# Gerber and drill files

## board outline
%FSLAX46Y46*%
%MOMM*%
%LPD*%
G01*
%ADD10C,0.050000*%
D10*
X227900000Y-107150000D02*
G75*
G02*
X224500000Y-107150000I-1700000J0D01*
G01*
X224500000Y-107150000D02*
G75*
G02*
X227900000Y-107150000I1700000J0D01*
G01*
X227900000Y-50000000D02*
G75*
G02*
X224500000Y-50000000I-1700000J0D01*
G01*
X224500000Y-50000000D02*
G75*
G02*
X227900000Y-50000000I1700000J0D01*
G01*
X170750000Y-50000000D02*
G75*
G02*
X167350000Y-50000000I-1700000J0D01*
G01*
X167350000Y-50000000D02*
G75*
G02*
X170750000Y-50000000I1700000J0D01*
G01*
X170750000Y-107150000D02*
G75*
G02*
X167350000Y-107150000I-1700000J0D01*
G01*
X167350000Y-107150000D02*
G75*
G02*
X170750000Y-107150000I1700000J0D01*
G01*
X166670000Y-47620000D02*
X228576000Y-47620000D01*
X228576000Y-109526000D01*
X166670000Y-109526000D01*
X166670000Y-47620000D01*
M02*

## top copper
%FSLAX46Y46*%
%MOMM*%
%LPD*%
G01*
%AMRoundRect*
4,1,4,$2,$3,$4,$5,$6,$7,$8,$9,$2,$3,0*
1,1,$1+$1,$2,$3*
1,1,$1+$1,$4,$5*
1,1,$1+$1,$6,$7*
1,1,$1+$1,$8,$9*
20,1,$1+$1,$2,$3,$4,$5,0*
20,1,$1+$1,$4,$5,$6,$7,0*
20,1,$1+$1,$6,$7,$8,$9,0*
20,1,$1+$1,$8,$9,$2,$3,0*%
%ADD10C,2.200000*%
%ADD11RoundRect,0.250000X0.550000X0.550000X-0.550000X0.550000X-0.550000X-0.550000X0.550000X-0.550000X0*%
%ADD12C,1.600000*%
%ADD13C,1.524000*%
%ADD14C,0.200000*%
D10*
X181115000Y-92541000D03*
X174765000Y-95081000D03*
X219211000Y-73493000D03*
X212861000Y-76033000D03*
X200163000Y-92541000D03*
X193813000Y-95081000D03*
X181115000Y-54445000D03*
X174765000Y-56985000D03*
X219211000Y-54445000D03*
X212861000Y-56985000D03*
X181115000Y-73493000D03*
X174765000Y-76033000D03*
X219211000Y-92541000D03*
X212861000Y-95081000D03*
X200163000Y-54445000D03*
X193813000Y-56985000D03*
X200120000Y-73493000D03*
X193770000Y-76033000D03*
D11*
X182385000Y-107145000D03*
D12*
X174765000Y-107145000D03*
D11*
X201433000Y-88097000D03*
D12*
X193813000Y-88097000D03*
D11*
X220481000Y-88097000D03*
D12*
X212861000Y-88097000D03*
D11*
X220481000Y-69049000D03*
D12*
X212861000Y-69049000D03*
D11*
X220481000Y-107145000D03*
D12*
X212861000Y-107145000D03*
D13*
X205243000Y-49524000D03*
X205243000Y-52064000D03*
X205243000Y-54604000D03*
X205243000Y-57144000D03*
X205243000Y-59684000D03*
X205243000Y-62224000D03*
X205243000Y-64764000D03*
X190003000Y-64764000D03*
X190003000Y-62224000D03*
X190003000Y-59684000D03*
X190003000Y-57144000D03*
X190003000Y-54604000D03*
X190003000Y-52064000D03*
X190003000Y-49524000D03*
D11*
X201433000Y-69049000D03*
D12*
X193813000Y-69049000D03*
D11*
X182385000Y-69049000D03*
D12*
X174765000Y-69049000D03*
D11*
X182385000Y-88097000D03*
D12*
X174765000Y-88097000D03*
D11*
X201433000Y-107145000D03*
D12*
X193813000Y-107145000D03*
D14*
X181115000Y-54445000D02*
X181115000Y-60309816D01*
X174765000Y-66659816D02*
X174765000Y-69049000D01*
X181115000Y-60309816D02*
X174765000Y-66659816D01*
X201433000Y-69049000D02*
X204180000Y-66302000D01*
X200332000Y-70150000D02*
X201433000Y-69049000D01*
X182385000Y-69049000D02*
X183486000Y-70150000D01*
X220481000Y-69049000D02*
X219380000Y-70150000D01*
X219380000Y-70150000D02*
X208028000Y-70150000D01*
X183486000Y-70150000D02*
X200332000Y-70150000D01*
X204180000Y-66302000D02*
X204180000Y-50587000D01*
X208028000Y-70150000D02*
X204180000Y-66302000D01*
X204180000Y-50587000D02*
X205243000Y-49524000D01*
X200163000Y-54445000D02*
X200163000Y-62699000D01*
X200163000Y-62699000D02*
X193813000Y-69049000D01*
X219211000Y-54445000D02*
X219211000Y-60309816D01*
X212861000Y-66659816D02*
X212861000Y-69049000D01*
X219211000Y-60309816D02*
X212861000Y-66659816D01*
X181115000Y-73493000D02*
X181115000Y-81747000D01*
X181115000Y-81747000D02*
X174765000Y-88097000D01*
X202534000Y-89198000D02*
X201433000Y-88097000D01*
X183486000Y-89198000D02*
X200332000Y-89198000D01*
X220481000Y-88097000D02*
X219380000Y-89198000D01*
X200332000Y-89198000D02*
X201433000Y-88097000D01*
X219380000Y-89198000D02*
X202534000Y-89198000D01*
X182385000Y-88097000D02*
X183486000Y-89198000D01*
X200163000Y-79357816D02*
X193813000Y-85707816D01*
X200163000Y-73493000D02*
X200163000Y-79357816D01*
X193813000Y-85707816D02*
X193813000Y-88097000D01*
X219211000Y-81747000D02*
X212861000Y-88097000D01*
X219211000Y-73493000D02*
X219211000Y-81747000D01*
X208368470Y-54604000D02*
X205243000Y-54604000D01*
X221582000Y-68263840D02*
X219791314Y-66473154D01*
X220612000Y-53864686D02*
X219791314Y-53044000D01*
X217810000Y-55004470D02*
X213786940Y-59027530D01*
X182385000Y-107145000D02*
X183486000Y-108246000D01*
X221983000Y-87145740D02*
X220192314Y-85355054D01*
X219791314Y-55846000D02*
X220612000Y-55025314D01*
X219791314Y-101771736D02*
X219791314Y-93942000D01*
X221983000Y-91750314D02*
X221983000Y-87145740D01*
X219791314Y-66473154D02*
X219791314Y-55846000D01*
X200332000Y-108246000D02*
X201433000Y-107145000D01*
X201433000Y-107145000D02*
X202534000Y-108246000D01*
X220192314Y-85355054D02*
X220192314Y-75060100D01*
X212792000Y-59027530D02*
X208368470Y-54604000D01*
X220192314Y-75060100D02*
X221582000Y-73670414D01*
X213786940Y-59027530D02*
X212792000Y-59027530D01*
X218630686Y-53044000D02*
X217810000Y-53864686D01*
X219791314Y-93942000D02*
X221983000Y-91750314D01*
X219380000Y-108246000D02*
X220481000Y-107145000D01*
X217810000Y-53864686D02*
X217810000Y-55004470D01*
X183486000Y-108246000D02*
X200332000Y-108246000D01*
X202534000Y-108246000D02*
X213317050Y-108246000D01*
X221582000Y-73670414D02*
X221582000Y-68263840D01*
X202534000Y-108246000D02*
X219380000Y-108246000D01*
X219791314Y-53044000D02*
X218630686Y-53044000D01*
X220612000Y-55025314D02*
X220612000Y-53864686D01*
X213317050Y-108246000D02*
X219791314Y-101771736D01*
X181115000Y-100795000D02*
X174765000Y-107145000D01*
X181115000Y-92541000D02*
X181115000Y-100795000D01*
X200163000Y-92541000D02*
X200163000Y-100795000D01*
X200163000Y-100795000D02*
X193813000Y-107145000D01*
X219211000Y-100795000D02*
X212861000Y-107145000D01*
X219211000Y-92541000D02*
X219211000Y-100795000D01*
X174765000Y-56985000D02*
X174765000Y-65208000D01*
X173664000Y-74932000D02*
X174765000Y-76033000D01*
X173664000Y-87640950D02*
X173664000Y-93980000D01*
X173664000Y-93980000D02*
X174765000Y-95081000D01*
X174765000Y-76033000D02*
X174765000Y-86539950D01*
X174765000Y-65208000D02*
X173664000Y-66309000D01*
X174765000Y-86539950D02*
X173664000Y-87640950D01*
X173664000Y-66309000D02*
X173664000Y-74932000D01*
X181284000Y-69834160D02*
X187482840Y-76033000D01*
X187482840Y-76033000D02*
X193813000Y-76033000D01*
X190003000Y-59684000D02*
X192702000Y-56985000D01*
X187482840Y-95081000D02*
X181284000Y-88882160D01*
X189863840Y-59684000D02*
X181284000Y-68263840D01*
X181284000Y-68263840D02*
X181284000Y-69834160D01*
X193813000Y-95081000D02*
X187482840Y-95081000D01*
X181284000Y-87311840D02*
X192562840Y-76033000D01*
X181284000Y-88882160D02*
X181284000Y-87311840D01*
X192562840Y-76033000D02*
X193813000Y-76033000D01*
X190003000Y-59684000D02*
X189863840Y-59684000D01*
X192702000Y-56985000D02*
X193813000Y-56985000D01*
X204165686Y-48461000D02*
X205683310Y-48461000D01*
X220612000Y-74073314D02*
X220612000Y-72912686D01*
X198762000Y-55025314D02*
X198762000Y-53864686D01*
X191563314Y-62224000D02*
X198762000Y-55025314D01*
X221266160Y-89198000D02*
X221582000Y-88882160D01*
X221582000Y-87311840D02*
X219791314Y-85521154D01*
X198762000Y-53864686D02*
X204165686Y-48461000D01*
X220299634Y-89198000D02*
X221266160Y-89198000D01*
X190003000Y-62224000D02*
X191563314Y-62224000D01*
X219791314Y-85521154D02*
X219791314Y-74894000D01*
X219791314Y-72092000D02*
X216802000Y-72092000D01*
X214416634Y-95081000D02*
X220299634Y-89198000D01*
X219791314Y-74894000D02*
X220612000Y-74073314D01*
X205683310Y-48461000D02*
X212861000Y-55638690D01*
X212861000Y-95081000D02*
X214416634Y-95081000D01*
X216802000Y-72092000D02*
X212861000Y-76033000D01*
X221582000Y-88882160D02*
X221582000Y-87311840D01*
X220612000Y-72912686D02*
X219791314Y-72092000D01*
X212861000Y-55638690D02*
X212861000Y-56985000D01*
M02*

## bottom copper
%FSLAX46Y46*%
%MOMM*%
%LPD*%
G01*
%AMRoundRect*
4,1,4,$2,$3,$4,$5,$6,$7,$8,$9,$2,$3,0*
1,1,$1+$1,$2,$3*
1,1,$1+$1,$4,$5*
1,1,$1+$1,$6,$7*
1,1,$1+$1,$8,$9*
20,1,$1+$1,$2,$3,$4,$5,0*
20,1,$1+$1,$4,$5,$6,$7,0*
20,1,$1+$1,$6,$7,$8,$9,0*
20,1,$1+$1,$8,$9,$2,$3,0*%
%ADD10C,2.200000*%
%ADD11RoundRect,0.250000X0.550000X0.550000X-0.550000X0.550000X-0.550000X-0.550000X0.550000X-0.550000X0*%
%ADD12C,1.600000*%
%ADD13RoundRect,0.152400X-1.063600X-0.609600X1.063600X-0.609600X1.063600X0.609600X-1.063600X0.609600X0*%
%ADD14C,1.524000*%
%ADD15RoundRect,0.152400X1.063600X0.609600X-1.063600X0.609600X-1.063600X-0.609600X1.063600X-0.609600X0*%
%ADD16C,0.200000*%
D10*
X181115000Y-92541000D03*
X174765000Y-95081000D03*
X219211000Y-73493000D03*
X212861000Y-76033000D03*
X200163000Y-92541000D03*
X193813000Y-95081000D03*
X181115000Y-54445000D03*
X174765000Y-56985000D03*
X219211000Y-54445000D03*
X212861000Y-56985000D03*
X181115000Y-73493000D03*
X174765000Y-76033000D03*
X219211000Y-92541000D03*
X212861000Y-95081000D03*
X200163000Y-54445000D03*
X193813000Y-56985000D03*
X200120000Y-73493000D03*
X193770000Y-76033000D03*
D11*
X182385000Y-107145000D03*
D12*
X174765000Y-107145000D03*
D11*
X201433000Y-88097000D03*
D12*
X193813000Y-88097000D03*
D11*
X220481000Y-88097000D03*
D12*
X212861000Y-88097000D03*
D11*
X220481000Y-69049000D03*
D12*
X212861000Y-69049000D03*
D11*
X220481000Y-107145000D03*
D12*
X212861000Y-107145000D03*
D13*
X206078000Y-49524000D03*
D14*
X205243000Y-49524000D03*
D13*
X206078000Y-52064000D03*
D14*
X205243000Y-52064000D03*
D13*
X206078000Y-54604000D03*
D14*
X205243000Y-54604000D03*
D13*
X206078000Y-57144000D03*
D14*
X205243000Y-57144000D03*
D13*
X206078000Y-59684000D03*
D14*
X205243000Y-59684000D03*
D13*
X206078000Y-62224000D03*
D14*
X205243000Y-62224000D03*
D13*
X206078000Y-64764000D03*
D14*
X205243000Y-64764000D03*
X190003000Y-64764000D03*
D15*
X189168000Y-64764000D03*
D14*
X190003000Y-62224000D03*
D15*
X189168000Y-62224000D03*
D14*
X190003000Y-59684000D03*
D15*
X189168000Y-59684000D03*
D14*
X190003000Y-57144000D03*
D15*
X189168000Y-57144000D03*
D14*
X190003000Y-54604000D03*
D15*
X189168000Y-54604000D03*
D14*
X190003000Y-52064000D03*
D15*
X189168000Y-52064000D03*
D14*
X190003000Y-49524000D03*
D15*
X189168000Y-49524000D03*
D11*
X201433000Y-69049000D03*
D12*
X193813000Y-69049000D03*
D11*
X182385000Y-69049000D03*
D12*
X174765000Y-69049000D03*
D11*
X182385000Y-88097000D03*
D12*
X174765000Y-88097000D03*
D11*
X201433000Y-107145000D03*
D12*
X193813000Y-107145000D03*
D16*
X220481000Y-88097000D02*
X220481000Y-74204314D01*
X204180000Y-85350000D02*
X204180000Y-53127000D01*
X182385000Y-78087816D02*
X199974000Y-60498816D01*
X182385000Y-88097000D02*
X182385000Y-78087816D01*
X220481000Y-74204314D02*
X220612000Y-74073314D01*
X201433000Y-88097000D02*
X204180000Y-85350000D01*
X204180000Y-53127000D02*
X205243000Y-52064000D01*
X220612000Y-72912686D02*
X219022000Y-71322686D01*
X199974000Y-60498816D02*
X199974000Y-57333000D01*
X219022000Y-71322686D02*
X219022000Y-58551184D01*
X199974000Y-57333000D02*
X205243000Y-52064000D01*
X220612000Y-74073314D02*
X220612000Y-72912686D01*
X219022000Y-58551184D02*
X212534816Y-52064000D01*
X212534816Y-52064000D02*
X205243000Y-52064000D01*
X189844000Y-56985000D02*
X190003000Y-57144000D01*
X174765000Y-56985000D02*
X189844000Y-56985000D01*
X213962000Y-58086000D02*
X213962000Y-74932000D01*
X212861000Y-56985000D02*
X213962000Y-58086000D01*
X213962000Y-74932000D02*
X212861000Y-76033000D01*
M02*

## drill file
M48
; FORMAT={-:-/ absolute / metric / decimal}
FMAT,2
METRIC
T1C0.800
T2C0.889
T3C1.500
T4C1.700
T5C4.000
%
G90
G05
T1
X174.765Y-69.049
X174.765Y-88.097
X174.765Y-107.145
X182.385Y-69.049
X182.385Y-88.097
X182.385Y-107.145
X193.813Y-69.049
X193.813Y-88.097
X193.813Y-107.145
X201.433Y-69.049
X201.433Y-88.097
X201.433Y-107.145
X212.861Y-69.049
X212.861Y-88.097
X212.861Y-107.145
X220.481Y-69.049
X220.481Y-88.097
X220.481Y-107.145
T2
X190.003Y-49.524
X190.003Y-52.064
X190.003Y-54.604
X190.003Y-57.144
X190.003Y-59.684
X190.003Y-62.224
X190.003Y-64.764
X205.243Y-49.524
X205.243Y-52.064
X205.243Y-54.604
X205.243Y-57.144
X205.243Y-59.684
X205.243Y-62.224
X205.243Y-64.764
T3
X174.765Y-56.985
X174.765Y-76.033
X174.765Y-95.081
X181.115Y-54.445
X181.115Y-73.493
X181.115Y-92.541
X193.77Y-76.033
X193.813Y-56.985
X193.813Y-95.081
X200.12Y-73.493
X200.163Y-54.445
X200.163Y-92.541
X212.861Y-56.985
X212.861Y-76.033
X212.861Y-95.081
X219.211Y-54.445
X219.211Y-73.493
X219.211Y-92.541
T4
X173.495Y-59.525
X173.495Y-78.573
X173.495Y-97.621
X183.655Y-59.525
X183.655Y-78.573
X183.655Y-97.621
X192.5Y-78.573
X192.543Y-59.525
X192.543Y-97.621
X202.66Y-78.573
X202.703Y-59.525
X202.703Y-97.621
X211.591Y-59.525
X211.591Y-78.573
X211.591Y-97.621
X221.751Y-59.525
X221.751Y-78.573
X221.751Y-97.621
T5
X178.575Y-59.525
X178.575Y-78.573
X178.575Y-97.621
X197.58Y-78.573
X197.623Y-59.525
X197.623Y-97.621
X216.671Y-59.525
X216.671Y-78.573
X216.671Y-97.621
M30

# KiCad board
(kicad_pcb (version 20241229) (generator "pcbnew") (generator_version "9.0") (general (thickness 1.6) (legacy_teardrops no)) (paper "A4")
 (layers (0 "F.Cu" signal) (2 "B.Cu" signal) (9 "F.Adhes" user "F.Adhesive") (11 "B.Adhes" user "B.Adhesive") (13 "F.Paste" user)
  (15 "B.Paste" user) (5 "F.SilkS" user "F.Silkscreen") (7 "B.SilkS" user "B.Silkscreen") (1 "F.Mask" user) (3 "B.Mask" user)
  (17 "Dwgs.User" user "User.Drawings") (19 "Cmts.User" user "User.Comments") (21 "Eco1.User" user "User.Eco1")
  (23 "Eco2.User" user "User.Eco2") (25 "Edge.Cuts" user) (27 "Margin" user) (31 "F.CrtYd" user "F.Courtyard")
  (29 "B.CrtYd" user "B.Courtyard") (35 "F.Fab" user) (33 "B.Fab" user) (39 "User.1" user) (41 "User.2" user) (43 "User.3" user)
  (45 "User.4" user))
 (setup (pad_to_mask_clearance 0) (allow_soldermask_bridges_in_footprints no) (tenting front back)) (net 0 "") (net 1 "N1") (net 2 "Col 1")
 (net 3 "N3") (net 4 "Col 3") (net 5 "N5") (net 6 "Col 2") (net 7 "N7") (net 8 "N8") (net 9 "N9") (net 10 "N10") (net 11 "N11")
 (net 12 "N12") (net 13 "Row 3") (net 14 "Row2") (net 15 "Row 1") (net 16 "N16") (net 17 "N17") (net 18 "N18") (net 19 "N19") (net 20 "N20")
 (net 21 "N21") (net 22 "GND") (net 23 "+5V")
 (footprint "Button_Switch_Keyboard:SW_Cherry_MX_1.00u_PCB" (layer "F.Cu") (at 181.115 92.541)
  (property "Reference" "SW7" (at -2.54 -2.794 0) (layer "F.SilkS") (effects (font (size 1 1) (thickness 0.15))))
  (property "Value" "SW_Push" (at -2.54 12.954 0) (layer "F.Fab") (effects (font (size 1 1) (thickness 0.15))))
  (pad "" np_thru_hole circle (at -7.62 5.08) (size 1.7 1.7) (drill 1.7) (layers "*.Cu" "*.Mask"))
  (pad "" np_thru_hole circle (at -2.54 5.08) (size 4 4) (drill 4) (layers "*.Cu" "*.Mask"))
  (pad "" np_thru_hole circle (at 2.54 5.08) (size 1.7 1.7) (drill 1.7) (layers "*.Cu" "*.Mask"))
  (pad "1" thru_hole circle (at 0 0) (size 2.2 2.2) (drill 1.5) (layers "*.Cu" "*.Mask") (remove_unused_layers no) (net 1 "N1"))
  (pad "2" thru_hole circle (at -6.35 2.54) (size 2.2 2.2) (drill 1.5) (layers "*.Cu" "*.Mask") (remove_unused_layers no) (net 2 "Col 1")))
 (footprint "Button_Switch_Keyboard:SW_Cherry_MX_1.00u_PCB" (layer "F.Cu") (at 219.211 73.493)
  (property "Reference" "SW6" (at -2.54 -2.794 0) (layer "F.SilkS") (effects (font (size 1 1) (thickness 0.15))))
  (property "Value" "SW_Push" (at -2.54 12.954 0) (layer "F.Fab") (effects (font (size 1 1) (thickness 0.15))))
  (pad "" np_thru_hole circle (at -7.62 5.08) (size 1.7 1.7) (drill 1.7) (layers "*.Cu" "*.Mask"))
  (pad "" np_thru_hole circle (at -2.54 5.08) (size 4 4) (drill 4) (layers "*.Cu" "*.Mask"))
  (pad "" np_thru_hole circle (at 2.54 5.08) (size 1.7 1.7) (drill 1.7) (layers "*.Cu" "*.Mask"))
  (pad "1" thru_hole circle (at 0 0) (size 2.2 2.2) (drill 1.5) (layers "*.Cu" "*.Mask") (remove_unused_layers no) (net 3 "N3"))
  (pad "2" thru_hole circle (at -6.35 2.54) (size 2.2 2.2) (drill 1.5) (layers "*.Cu" "*.Mask") (remove_unused_layers no) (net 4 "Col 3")))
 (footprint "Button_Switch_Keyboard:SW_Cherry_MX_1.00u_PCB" (layer "F.Cu") (at 200.163 92.541)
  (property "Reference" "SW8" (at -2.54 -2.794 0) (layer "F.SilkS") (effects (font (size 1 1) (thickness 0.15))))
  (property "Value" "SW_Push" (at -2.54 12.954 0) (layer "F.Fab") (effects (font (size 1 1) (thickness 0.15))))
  (pad "" np_thru_hole circle (at -7.62 5.08) (size 1.7 1.7) (drill 1.7) (layers "*.Cu" "*.Mask"))
  (pad "" np_thru_hole circle (at -2.54 5.08) (size 4 4) (drill 4) (layers "*.Cu" "*.Mask"))
  (pad "" np_thru_hole circle (at 2.54 5.08) (size 1.7 1.7) (drill 1.7) (layers "*.Cu" "*.Mask"))
  (pad "1" thru_hole circle (at 0 0) (size 2.2 2.2) (drill 1.5) (layers "*.Cu" "*.Mask") (remove_unused_layers no) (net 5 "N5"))
  (pad "2" thru_hole circle (at -6.35 2.54) (size 2.2 2.2) (drill 1.5) (layers "*.Cu" "*.Mask") (remove_unused_layers no) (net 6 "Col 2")))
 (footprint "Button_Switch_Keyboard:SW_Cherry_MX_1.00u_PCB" (layer "F.Cu") (at 181.115 54.445)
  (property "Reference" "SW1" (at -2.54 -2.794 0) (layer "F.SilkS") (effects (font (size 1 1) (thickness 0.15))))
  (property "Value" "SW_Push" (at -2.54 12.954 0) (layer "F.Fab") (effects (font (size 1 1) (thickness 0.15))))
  (pad "" np_thru_hole circle (at -7.62 5.08) (size 1.7 1.7) (drill 1.7) (layers "*.Cu" "*.Mask"))
  (pad "" np_thru_hole circle (at -2.54 5.08) (size 4 4) (drill 4) (layers "*.Cu" "*.Mask"))
  (pad "" np_thru_hole circle (at 2.54 5.08) (size 1.7 1.7) (drill 1.7) (layers "*.Cu" "*.Mask"))
  (pad "1" thru_hole circle (at 0 0) (size 2.2 2.2) (drill 1.5) (layers "*.Cu" "*.Mask") (remove_unused_layers no) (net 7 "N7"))
  (pad "2" thru_hole circle (at -6.35 2.54) (size 2.2 2.2) (drill 1.5) (layers "*.Cu" "*.Mask") (remove_unused_layers no) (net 2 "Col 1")))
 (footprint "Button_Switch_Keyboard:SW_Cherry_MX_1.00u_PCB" (layer "F.Cu") (at 219.211 54.445)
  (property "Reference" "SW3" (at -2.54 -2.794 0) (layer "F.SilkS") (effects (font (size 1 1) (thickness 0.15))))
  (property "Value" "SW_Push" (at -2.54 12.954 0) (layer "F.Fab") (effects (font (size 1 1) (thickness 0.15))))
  (pad "" np_thru_hole circle (at -7.62 5.08) (size 1.7 1.7) (drill 1.7) (layers "*.Cu" "*.Mask"))
  (pad "" np_thru_hole circle (at -2.54 5.08) (size 4 4) (drill 4) (layers "*.Cu" "*.Mask"))
  (pad "" np_thru_hole circle (at 2.54 5.08) (size 1.7 1.7) (drill 1.7) (layers "*.Cu" "*.Mask"))
  (pad "1" thru_hole circle (at 0 0) (size 2.2 2.2) (drill 1.5) (layers "*.Cu" "*.Mask") (remove_unused_layers no) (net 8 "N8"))
  (pad "2" thru_hole circle (at -6.35 2.54) (size 2.2 2.2) (drill 1.5) (layers "*.Cu" "*.Mask") (remove_unused_layers no) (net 4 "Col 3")))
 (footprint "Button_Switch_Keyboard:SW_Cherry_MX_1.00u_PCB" (layer "F.Cu") (at 181.115 73.493)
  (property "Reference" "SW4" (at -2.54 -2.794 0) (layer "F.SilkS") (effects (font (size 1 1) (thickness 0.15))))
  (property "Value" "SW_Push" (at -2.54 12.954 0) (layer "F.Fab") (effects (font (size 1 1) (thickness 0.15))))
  (pad "" np_thru_hole circle (at -7.62 5.08) (size 1.7 1.7) (drill 1.7) (layers "*.Cu" "*.Mask"))
  (pad "" np_thru_hole circle (at -2.54 5.08) (size 4 4) (drill 4) (layers "*.Cu" "*.Mask"))
  (pad "" np_thru_hole circle (at 2.54 5.08) (size 1.7 1.7) (drill 1.7) (layers "*.Cu" "*.Mask"))
  (pad "1" thru_hole circle (at 0 0) (size 2.2 2.2) (drill 1.5) (layers "*.Cu" "*.Mask") (remove_unused_layers no) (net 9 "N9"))
  (pad "2" thru_hole circle (at -6.35 2.54) (size 2.2 2.2) (drill 1.5) (layers "*.Cu" "*.Mask") (remove_unused_layers no) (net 2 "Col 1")))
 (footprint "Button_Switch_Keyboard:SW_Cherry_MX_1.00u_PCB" (layer "F.Cu") (at 219.211 92.541)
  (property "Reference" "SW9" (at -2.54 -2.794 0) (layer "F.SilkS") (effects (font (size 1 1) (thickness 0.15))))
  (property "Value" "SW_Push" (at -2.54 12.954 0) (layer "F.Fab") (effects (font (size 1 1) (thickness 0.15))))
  (pad "" np_thru_hole circle (at -7.62 5.08) (size 1.7 1.7) (drill 1.7) (layers "*.Cu" "*.Mask"))
  (pad "" np_thru_hole circle (at -2.54 5.08) (size 4 4) (drill 4) (layers "*.Cu" "*.Mask"))
  (pad "" np_thru_hole circle (at 2.54 5.08) (size 1.7 1.7) (drill 1.7) (layers "*.Cu" "*.Mask"))
  (pad "1" thru_hole circle (at 0 0) (size 2.2 2.2) (drill 1.5) (layers "*.Cu" "*.Mask") (remove_unused_layers no) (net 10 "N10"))
  (pad "2" thru_hole circle (at -6.35 2.54) (size 2.2 2.2) (drill 1.5) (layers "*.Cu" "*.Mask") (remove_unused_layers no) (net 4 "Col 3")))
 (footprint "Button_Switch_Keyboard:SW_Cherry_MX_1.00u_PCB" (layer "F.Cu") (at 200.163 54.445)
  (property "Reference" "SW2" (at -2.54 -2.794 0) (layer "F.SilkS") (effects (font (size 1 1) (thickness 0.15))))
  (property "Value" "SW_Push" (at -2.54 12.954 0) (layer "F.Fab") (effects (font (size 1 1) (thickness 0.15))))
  (pad "" np_thru_hole circle (at -7.62 5.08) (size 1.7 1.7) (drill 1.7) (layers "*.Cu" "*.Mask"))
  (pad "" np_thru_hole circle (at -2.54 5.08) (size 4 4) (drill 4) (layers "*.Cu" "*.Mask"))
  (pad "" np_thru_hole circle (at 2.54 5.08) (size 1.7 1.7) (drill 1.7) (layers "*.Cu" "*.Mask"))
  (pad "1" thru_hole circle (at 0 0) (size 2.2 2.2) (drill 1.5) (layers "*.Cu" "*.Mask") (remove_unused_layers no) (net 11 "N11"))
  (pad "2" thru_hole circle (at -6.35 2.54) (size 2.2 2.2) (drill 1.5) (layers "*.Cu" "*.Mask") (remove_unused_layers no) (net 6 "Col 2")))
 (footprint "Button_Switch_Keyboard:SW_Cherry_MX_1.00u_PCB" (layer "F.Cu") (at 200.12 73.493)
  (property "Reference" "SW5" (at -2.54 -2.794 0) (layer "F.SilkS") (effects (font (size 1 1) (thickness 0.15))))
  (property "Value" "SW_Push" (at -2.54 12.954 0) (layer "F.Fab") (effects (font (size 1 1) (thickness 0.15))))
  (pad "" np_thru_hole circle (at -7.62 5.08) (size 1.7 1.7) (drill 1.7) (layers "*.Cu" "*.Mask"))
  (pad "" np_thru_hole circle (at -2.54 5.08) (size 4 4) (drill 4) (layers "*.Cu" "*.Mask"))
  (pad "" np_thru_hole circle (at 2.54 5.08) (size 1.7 1.7) (drill 1.7) (layers "*.Cu" "*.Mask"))
  (pad "1" thru_hole circle (at 0 0) (size 2.2 2.2) (drill 1.5) (layers "*.Cu" "*.Mask") (remove_unused_layers no) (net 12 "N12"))
  (pad "2" thru_hole circle (at -6.35 2.54) (size 2.2 2.2) (drill 1.5) (layers "*.Cu" "*.Mask") (remove_unused_layers no) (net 6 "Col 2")))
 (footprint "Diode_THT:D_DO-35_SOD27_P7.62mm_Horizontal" (layer "B.Cu") (at 182.385 107.145 180)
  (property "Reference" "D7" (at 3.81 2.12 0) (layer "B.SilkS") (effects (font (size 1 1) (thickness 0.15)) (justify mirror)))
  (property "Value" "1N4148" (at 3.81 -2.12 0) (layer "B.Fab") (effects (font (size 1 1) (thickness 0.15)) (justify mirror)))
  (pad "1" thru_hole roundrect (at 0 0 180) (size 1.6 1.6) (drill 0.8) (layers "*.Cu" "*.Mask") (remove_unused_layers no)
   (roundrect_rratio 0.15625) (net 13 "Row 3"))
  (pad "2" thru_hole circle (at 7.62 0 180) (size 1.6 1.6) (drill 0.8) (layers "*.Cu" "*.Mask") (remove_unused_layers no) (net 1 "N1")))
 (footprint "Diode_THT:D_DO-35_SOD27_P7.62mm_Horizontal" (layer "B.Cu") (at 201.433 88.097 180)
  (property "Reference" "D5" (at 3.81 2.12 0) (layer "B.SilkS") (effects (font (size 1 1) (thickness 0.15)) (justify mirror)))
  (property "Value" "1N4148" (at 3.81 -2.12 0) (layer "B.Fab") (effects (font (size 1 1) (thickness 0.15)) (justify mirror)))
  (pad "1" thru_hole roundrect (at 0 0 180) (size 1.6 1.6) (drill 0.8) (layers "*.Cu" "*.Mask") (remove_unused_layers no)
   (roundrect_rratio 0.15625) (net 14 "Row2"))
  (pad "2" thru_hole circle (at 7.62 0 180) (size 1.6 1.6) (drill 0.8) (layers "*.Cu" "*.Mask") (remove_unused_layers no) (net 12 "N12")))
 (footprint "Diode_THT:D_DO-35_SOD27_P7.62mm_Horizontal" (layer "B.Cu") (at 220.481 88.097 180)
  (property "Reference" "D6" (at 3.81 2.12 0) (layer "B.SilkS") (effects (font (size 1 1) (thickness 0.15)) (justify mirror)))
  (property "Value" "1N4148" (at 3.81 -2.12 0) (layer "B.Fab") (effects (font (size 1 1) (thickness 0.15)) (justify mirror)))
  (pad "1" thru_hole roundrect (at 0 0 180) (size 1.6 1.6) (drill 0.8) (layers "*.Cu" "*.Mask") (remove_unused_layers no)
   (roundrect_rratio 0.15625) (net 14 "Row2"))
  (pad "2" thru_hole circle (at 7.62 0 180) (size 1.6 1.6) (drill 0.8) (layers "*.Cu" "*.Mask") (remove_unused_layers no) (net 3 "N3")))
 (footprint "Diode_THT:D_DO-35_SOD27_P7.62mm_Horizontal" (layer "B.Cu") (at 220.481 69.049 180)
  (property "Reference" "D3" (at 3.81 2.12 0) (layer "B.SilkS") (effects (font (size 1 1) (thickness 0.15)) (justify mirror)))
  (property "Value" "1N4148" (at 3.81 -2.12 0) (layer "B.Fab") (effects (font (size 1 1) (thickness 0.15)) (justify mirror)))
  (pad "1" thru_hole roundrect (at 0 0 180) (size 1.6 1.6) (drill 0.8) (layers "*.Cu" "*.Mask") (remove_unused_layers no)
   (roundrect_rratio 0.15625) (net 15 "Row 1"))
  (pad "2" thru_hole circle (at 7.62 0 180) (size 1.6 1.6) (drill 0.8) (layers "*.Cu" "*.Mask") (remove_unused_layers no) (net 8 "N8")))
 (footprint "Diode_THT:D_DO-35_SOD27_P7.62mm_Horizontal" (layer "B.Cu") (at 220.481 107.145 180)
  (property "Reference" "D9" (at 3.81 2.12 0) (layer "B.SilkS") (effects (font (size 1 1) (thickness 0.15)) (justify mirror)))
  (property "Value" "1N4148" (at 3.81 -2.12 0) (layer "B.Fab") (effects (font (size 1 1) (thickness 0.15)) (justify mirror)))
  (pad "1" thru_hole roundrect (at 0 0 180) (size 1.6 1.6) (drill 0.8) (layers "*.Cu" "*.Mask") (remove_unused_layers no)
   (roundrect_rratio 0.15625) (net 13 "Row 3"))
  (pad "2" thru_hole circle (at 7.62 0 180) (size 1.6 1.6) (drill 0.8) (layers "*.Cu" "*.Mask") (remove_unused_layers no) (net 10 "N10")))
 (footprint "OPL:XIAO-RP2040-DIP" (layer "B.Cu") (at 197.623 57.144 180)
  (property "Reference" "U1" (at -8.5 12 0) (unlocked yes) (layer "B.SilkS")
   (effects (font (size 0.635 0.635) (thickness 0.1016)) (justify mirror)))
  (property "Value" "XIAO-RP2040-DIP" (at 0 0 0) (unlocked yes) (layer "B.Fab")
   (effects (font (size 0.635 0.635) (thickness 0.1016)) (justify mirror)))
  (pad "1" smd roundrect (at -8.455 7.62) (size 2.432 1.524) (layers "B.Cu" "B.Mask") (roundrect_rratio 0.1) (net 15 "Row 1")
   (thermal_bridge_angle 45))
  (pad "1" thru_hole circle (at -7.62 7.62) (size 1.524 1.524) (drill 0.889) (layers "*.Cu" "*.Mask") (remove_unused_layers no)
   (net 15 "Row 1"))
  (pad "2" smd roundrect (at -8.455 5.08) (size 2.432 1.524) (layers "B.Cu" "B.Mask") (roundrect_rratio 0.1) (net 14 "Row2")
   (thermal_bridge_angle 45))
  (pad "2" thru_hole circle (at -7.62 5.08) (size 1.524 1.524) (drill 0.889) (layers "*.Cu" "*.Mask") (remove_unused_layers no)
   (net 14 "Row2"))
  (pad "3" smd roundrect (at -8.455 2.54) (size 2.432 1.524) (layers "B.Cu" "B.Mask") (roundrect_rratio 0.1) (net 13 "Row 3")
   (thermal_bridge_angle 45))
  (pad "3" thru_hole circle (at -7.62 2.54) (size 1.524 1.524) (drill 0.889) (layers "*.Cu" "*.Mask") (remove_unused_layers no)
   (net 13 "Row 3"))
  (pad "4" smd roundrect (at -8.455 0) (size 2.432 1.524) (layers "B.Cu" "B.Mask") (roundrect_rratio 0.1) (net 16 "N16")
   (thermal_bridge_angle 45))
  (pad "4" thru_hole circle (at -7.62 0) (size 1.524 1.524) (drill 0.889) (layers "*.Cu" "*.Mask") (remove_unused_layers no) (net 16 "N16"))
  (pad "5" smd roundrect (at -8.455 -2.54) (size 2.432 1.524) (layers "B.Cu" "B.Mask") (roundrect_rratio 0.1) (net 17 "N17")
   (thermal_bridge_angle 45))
  (pad "5" thru_hole circle (at -7.62 -2.54) (size 1.524 1.524) (drill 0.889) (layers "*.Cu" "*.Mask") (remove_unused_layers no)
   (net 17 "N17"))
  (pad "6" smd roundrect (at -8.455 -5.08) (size 2.432 1.524) (layers "B.Cu" "B.Mask") (roundrect_rratio 0.1) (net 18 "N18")
   (thermal_bridge_angle 45))
  (pad "6" thru_hole circle (at -7.62 -5.08) (size 1.524 1.524) (drill 0.889) (layers "*.Cu" "*.Mask") (remove_unused_layers no)
   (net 18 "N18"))
  (pad "7" smd roundrect (at -8.455 -7.62) (size 2.432 1.524) (layers "B.Cu" "B.Mask") (roundrect_rratio 0.1) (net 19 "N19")
   (thermal_bridge_angle 45))
  (pad "7" thru_hole circle (at -7.62 -7.62) (size 1.524 1.524) (drill 0.889) (layers "*.Cu" "*.Mask") (remove_unused_layers no)
   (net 19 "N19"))
  (pad "8" thru_hole circle (at 7.62 -7.62 180) (size 1.524 1.524) (drill 0.889) (layers "*.Cu" "*.Mask") (remove_unused_layers no)
   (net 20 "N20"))
  (pad "8" smd roundrect (at 8.455 -7.62 180) (size 2.432 1.524) (layers "B.Cu" "B.Mask") (roundrect_rratio 0.1) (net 20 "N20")
   (thermal_bridge_angle 45))
  (pad "9" thru_hole circle (at 7.62 -5.08 180) (size 1.524 1.524) (drill 0.889) (layers "*.Cu" "*.Mask") (remove_unused_layers no)
   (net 4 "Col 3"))
  (pad "9" smd roundrect (at 8.455 -5.08 180) (size 2.432 1.524) (layers "B.Cu" "B.Mask") (roundrect_rratio 0.1) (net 4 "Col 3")
   (thermal_bridge_angle 45))
  (pad "10" thru_hole circle (at 7.62 -2.54 180) (size 1.524 1.524) (drill 0.889) (layers "*.Cu" "*.Mask") (remove_unused_layers no)
   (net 6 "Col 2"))
  (pad "10" smd roundrect (at 8.455 -2.54 180) (size 2.432 1.524) (layers "B.Cu" "B.Mask") (roundrect_rratio 0.1) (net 6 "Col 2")
   (thermal_bridge_angle 45))
  (pad "11" thru_hole circle (at 7.62 0 180) (size 1.524 1.524) (drill 0.889) (layers "*.Cu" "*.Mask") (remove_unused_layers no)
   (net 2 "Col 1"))
  (pad "11" smd roundrect (at 8.455 0 180) (size 2.432 1.524) (layers "B.Cu" "B.Mask") (roundrect_rratio 0.1) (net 2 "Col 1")
   (thermal_bridge_angle 45))
  (pad "12" thru_hole circle (at 7.62 2.54 180) (size 1.524 1.524) (drill 0.889) (layers "*.Cu" "*.Mask") (remove_unused_layers no)
   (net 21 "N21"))
  (pad "12" smd roundrect (at 8.455 2.54 180) (size 2.432 1.524) (layers "B.Cu" "B.Mask") (roundrect_rratio 0.1) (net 21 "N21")
   (thermal_bridge_angle 45))
  (pad "13" thru_hole circle (at 7.62 5.08 180) (size 1.524 1.524) (drill 0.889) (layers "*.Cu" "*.Mask") (remove_unused_layers no)
   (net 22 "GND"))
  (pad "13" smd roundrect (at 8.455 5.08 180) (size 2.432 1.524) (layers "B.Cu" "B.Mask") (roundrect_rratio 0.1) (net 22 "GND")
   (thermal_bridge_angle 45))
  (pad "14" thru_hole circle (at 7.62 7.62 180) (size 1.524 1.524) (drill 0.889) (layers "*.Cu" "*.Mask") (remove_unused_layers no)
   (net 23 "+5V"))
  (pad "14" smd roundrect (at 8.455 7.62 180) (size 2.432 1.524) (layers "B.Cu" "B.Mask") (roundrect_rratio 0.1) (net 23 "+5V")
   (thermal_bridge_angle 45)))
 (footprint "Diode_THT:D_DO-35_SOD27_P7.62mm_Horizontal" (layer "B.Cu") (at 201.433 69.049 180)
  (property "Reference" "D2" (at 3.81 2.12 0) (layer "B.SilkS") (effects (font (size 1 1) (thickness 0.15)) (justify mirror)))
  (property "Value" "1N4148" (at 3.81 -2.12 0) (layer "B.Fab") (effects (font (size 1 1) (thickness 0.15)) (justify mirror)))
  (pad "1" thru_hole roundrect (at 0 0 180) (size 1.6 1.6) (drill 0.8) (layers "*.Cu" "*.Mask") (remove_unused_layers no)
   (roundrect_rratio 0.15625) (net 15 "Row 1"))
  (pad "2" thru_hole circle (at 7.62 0 180) (size 1.6 1.6) (drill 0.8) (layers "*.Cu" "*.Mask") (remove_unused_layers no) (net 11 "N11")))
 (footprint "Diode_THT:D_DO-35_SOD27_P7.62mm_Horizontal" (layer "B.Cu") (at 182.385 69.049 180)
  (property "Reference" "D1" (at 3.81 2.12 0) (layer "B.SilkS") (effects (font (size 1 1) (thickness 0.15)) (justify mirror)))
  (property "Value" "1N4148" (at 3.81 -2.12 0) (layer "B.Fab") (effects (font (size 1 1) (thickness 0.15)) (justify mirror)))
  (pad "1" thru_hole roundrect (at 0 0 180) (size 1.6 1.6) (drill 0.8) (layers "*.Cu" "*.Mask") (remove_unused_layers no)
   (roundrect_rratio 0.15625) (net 15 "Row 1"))
  (pad "2" thru_hole circle (at 7.62 0 180) (size 1.6 1.6) (drill 0.8) (layers "*.Cu" "*.Mask") (remove_unused_layers no) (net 7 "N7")))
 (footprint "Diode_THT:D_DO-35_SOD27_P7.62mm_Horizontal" (layer "B.Cu") (at 182.385 88.097 180)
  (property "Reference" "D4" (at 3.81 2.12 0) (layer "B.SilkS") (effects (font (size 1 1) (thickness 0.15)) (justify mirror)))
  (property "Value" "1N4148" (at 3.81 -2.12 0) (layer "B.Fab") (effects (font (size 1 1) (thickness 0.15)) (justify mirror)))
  (pad "1" thru_hole roundrect (at 0 0 180) (size 1.6 1.6) (drill 0.8) (layers "*.Cu" "*.Mask") (remove_unused_layers no)
   (roundrect_rratio 0.15625) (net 14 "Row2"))
  (pad "2" thru_hole circle (at 7.62 0 180) (size 1.6 1.6) (drill 0.8) (layers "*.Cu" "*.Mask") (remove_unused_layers no) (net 9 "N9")))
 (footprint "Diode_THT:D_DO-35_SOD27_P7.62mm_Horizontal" (layer "B.Cu") (at 201.433 107.145 180)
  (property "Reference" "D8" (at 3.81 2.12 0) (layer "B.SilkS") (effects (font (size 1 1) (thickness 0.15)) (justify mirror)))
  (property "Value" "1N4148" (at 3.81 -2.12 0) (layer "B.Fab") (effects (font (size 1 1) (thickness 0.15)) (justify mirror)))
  (pad "1" thru_hole roundrect (at 0 0 180) (size 1.6 1.6) (drill 0.8) (layers "*.Cu" "*.Mask") (remove_unused_layers no)
   (roundrect_rratio 0.15625) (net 13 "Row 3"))
  (pad "2" thru_hole circle (at 7.62 0 180) (size 1.6 1.6) (drill 0.8) (layers "*.Cu" "*.Mask") (remove_unused_layers no) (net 5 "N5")))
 (gr_circle (center 226.2 107.15) (end 224.5 107.15) (stroke (width 0.05) (type default)) (fill no) (layer "Edge.Cuts"))
 (gr_circle (center 226.2 50) (end 224.5 50) (stroke (width 0.05) (type default)) (fill no) (layer "Edge.Cuts"))
 (gr_circle (center 169.05 50) (end 170.75 50) (stroke (width 0.05) (type default)) (fill no) (layer "Edge.Cuts"))
 (gr_circle (center 169.05 107.15) (end 170.75 107.15) (stroke (width 0.05) (type default)) (fill no) (layer "Edge.Cuts"))
 (gr_rect (start 166.67 47.62) (end 228.576 109.526) (stroke (width 0.05) (type default)) (fill no) (layer "Edge.Cuts"))
 (segment (start 181.115 54.445) (end 181.115 60.309816) (width 0.2) (layer "F.Cu") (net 7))
 (segment (start 174.765 66.659816) (end 174.765 69.049) (width 0.2) (layer "F.Cu") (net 7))
 (segment (start 181.115 60.309816) (end 174.765 66.659816) (width 0.2) (layer "F.Cu") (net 7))
 (segment (start 201.433 69.049) (end 204.18 66.302) (width 0.2) (layer "F.Cu") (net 15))
 (segment (start 200.332 70.15) (end 201.433 69.049) (width 0.2) (layer "F.Cu") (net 15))
 (segment (start 182.385 69.049) (end 183.486 70.15) (width 0.2) (layer "F.Cu") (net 15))
 (segment (start 220.481 69.049) (end 219.38 70.15) (width 0.2) (layer "F.Cu") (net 15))
 (segment (start 219.38 70.15) (end 208.028 70.15) (width 0.2) (layer "F.Cu") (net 15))
 (segment (start 183.486 70.15) (end 200.332 70.15) (width 0.2) (layer "F.Cu") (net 15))
 (segment (start 204.18 66.302) (end 204.18 50.587) (width 0.2) (layer "F.Cu") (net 15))
 (segment (start 208.028 70.15) (end 204.18 66.302) (width 0.2) (layer "F.Cu") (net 15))
 (segment (start 204.18 50.587) (end 205.243 49.524) (width 0.2) (layer "F.Cu") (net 15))
 (segment (start 200.163 54.445) (end 200.163 62.699) (width 0.2) (layer "F.Cu") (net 11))
 (segment (start 200.163 62.699) (end 193.813 69.049) (width 0.2) (layer "F.Cu") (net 11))
 (segment (start 219.211 54.445) (end 219.211 60.309816) (width 0.2) (layer "F.Cu") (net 8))
 (segment (start 212.861 66.659816) (end 212.861 69.049) (width 0.2) (layer "F.Cu") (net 8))
 (segment (start 219.211 60.309816) (end 212.861 66.659816) (width 0.2) (layer "F.Cu") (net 8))
 (segment (start 181.115 73.493) (end 181.115 81.747) (width 0.2) (layer "F.Cu") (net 9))
 (segment (start 181.115 81.747) (end 174.765 88.097) (width 0.2) (layer "F.Cu") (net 9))
 (segment (start 202.534 89.198) (end 201.433 88.097) (width 0.2) (layer "F.Cu") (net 14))
 (segment (start 183.486 89.198) (end 200.332 89.198) (width 0.2) (layer "F.Cu") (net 14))
 (segment (start 220.481 88.097) (end 219.38 89.198) (width 0.2) (layer "F.Cu") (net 14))
 (segment (start 200.332 89.198) (end 201.433 88.097) (width 0.2) (layer "F.Cu") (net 14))
 (segment (start 219.38 89.198) (end 202.534 89.198) (width 0.2) (layer "F.Cu") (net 14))
 (segment (start 182.385 88.097) (end 183.486 89.198) (width 0.2) (layer "F.Cu") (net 14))
 (segment (start 220.481 88.097) (end 220.481 74.204314) (width 0.2) (layer "B.Cu") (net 14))
 (segment (start 204.18 85.35) (end 204.18 53.127) (width 0.2) (layer "B.Cu") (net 14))
 (segment (start 182.385 78.087816) (end 199.974 60.498816) (width 0.2) (layer "B.Cu") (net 14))
 (segment (start 182.385 88.097) (end 182.385 78.087816) (width 0.2) (layer "B.Cu") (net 14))
 (segment (start 220.481 74.204314) (end 220.612 74.073314) (width 0.2) (layer "B.Cu") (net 14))
 (segment (start 201.433 88.097) (end 204.18 85.35) (width 0.2) (layer "B.Cu") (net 14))
 (segment (start 204.18 53.127) (end 205.243 52.064) (width 0.2) (layer "B.Cu") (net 14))
 (segment (start 220.612 72.912686) (end 219.022 71.322686) (width 0.2) (layer "B.Cu") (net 14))
 (segment (start 199.974 60.498816) (end 199.974 57.333) (width 0.2) (layer "B.Cu") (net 14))
 (segment (start 219.022 71.322686) (end 219.022 58.551184) (width 0.2) (layer "B.Cu") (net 14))
 (segment (start 199.974 57.333) (end 205.243 52.064) (width 0.2) (layer "B.Cu") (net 14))
 (segment (start 220.612 74.073314) (end 220.612 72.912686) (width 0.2) (layer "B.Cu") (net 14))
 (segment (start 219.022 58.551184) (end 212.534816 52.064) (width 0.2) (layer "B.Cu") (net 14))
 (segment (start 212.534816 52.064) (end 205.243 52.064) (width 0.2) (layer "B.Cu") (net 14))
 (segment (start 200.163 79.357816) (end 193.813 85.707816) (width 0.2) (layer "F.Cu") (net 12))
 (segment (start 200.163 73.493) (end 200.163 79.357816) (width 0.2) (layer "F.Cu") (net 12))
 (segment (start 193.813 85.707816) (end 193.813 88.097) (width 0.2) (layer "F.Cu") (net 12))
 (segment (start 219.211 81.747) (end 212.861 88.097) (width 0.2) (layer "F.Cu") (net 3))
 (segment (start 219.211 73.493) (end 219.211 81.747) (width 0.2) (layer "F.Cu") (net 3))
 (segment (start 208.36847 54.604) (end 205.243 54.604) (width 0.2) (layer "F.Cu") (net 13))
 (segment (start 221.582 68.26384) (end 219.791314 66.473154) (width 0.2) (layer "F.Cu") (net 13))
 (segment (start 220.612 53.864686) (end 219.791314 53.044) (width 0.2) (layer "F.Cu") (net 13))
 (segment (start 217.81 55.00447) (end 213.78694 59.02753) (width 0.2) (layer "F.Cu") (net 13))
 (segment (start 182.385 107.145) (end 183.486 108.246) (width 0.2) (layer "F.Cu") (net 13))
 (segment (start 221.983 87.14574) (end 220.192314 85.355054) (width 0.2) (layer "F.Cu") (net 13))
 (segment (start 219.791314 55.846) (end 220.612 55.025314) (width 0.2) (layer "F.Cu") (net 13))
 (segment (start 219.791314 101.771736) (end 219.791314 93.942) (width 0.2) (layer "F.Cu") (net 13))
 (segment (start 221.983 91.750314) (end 221.983 87.14574) (width 0.2) (layer "F.Cu") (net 13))
 (segment (start 219.791314 66.473154) (end 219.791314 55.846) (width 0.2) (layer "F.Cu") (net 13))
 (segment (start 200.332 108.246) (end 201.433 107.145) (width 0.2) (layer "F.Cu") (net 13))
 (segment (start 201.433 107.145) (end 202.534 108.246) (width 0.2) (layer "F.Cu") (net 13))
 (segment (start 220.192314 85.355054) (end 220.192314 75.0601) (width 0.2) (layer "F.Cu") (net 13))
 (segment (start 212.792 59.02753) (end 208.36847 54.604) (width 0.2) (layer "F.Cu") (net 13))
 (segment (start 220.192314 75.0601) (end 221.582 73.670414) (width 0.2) (layer "F.Cu") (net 13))
 (segment (start 213.78694 59.02753) (end 212.792 59.02753) (width 0.2) (layer "F.Cu") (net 13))
 (segment (start 218.630686 53.044) (end 217.81 53.864686) (width 0.2) (layer "F.Cu") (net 13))
 (segment (start 219.791314 93.942) (end 221.983 91.750314) (width 0.2) (layer "F.Cu") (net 13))
 (segment (start 219.38 108.246) (end 220.481 107.145) (width 0.2) (layer "F.Cu") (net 13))
 (segment (start 217.81 53.864686) (end 217.81 55.00447) (width 0.2) (layer "F.Cu") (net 13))
 (segment (start 183.486 108.246) (end 200.332 108.246) (width 0.2) (layer "F.Cu") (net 13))
 (segment (start 202.534 108.246) (end 213.31705 108.246) (width 0.2) (layer "F.Cu") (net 13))
 (segment (start 221.582 73.670414) (end 221.582 68.26384) (width 0.2) (layer "F.Cu") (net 13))
 (segment (start 202.534 108.246) (end 219.38 108.246) (width 0.2) (layer "F.Cu") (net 13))
 (segment (start 219.791314 53.044) (end 218.630686 53.044) (width 0.2) (layer "F.Cu") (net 13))
 (segment (start 220.612 55.025314) (end 220.612 53.864686) (width 0.2) (layer "F.Cu") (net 13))
 (segment (start 213.31705 108.246) (end 219.791314 101.771736) (width 0.2) (layer "F.Cu") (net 13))
 (segment (start 181.115 100.795) (end 174.765 107.145) (width 0.2) (layer "F.Cu") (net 1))
 (segment (start 181.115 92.541) (end 181.115 100.795) (width 0.2) (layer "F.Cu") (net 1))
 (segment (start 200.163 92.541) (end 200.163 100.795) (width 0.2) (layer "F.Cu") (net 5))
 (segment (start 200.163 100.795) (end 193.813 107.145) (width 0.2) (layer "F.Cu") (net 5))
 (segment (start 219.211 100.795) (end 212.861 107.145) (width 0.2) (layer "F.Cu") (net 10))
 (segment (start 219.211 92.541) (end 219.211 100.795) (width 0.2) (layer "F.Cu") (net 10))
 (segment (start 174.765 56.985) (end 174.765 65.208) (width 0.2) (layer "F.Cu") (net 2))
 (segment (start 173.664 74.932) (end 174.765 76.033) (width 0.2) (layer "F.Cu") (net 2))
 (segment (start 173.664 87.64095) (end 173.664 93.98) (width 0.2) (layer "F.Cu") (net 2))
 (segment (start 173.664 93.98) (end 174.765 95.081) (width 0.2) (layer "F.Cu") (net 2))
 (segment (start 174.765 76.033) (end 174.765 86.53995) (width 0.2) (layer "F.Cu") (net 2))
 (segment (start 174.765 65.208) (end 173.664 66.309) (width 0.2) (layer "F.Cu") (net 2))
 (segment (start 174.765 86.53995) (end 173.664 87.64095) (width 0.2) (layer "F.Cu") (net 2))
 (segment (start 173.664 66.309) (end 173.664 74.932) (width 0.2) (layer "F.Cu") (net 2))
 (segment (start 189.844 56.985) (end 190.003 57.144) (width 0.2) (layer "B.Cu") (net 2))
 (segment (start 174.765 56.985) (end 189.844 56.985) (width 0.2) (layer "B.Cu") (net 2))
 (segment (start 181.284 69.83416) (end 187.48284 76.033) (width 0.2) (layer "F.Cu") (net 6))
 (segment (start 187.48284 76.033) (end 193.813 76.033) (width 0.2) (layer "F.Cu") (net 6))
 (segment (start 190.003 59.684) (end 192.702 56.985) (width 0.2) (layer "F.Cu") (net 6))
 (segment (start 187.48284 95.081) (end 181.284 88.88216) (width 0.2) (layer "F.Cu") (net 6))
 (segment (start 189.86384 59.684) (end 181.284 68.26384) (width 0.2) (layer "F.Cu") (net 6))
 (segment (start 181.284 68.26384) (end 181.284 69.83416) (width 0.2) (layer "F.Cu") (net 6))
 (segment (start 193.813 95.081) (end 187.48284 95.081) (width 0.2) (layer "F.Cu") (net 6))
 (segment (start 181.284 87.31184) (end 192.56284 76.033) (width 0.2) (layer "F.Cu") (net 6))
 (segment (start 181.284 88.88216) (end 181.284 87.31184) (width 0.2) (layer "F.Cu") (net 6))
 (segment (start 192.56284 76.033) (end 193.813 76.033) (width 0.2) (layer "F.Cu") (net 6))
 (segment (start 190.003 59.684) (end 189.86384 59.684) (width 0.2) (layer "F.Cu") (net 6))
 (segment (start 192.702 56.985) (end 193.813 56.985) (width 0.2) (layer "F.Cu") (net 6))
 (segment (start 204.165686 48.461) (end 205.68331 48.461) (width 0.2) (layer "F.Cu") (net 4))
 (segment (start 220.612 74.073314) (end 220.612 72.912686) (width 0.2) (layer "F.Cu") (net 4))
 (segment (start 198.762 55.025314) (end 198.762 53.864686) (width 0.2) (layer "F.Cu") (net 4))
 (segment (start 191.563314 62.224) (end 198.762 55.025314) (width 0.2) (layer "F.Cu") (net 4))
 (segment (start 221.26616 89.198) (end 221.582 88.88216) (width 0.2) (layer "F.Cu") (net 4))
 (segment (start 221.582 87.31184) (end 219.791314 85.521154) (width 0.2) (layer "F.Cu") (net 4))
 (segment (start 198.762 53.864686) (end 204.165686 48.461) (width 0.2) (layer "F.Cu") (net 4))
 (segment (start 220.299634 89.198) (end 221.26616 89.198) (width 0.2) (layer "F.Cu") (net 4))
 (segment (start 190.003 62.224) (end 191.563314 62.224) (width 0.2) (layer "F.Cu") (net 4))
 (segment (start 219.791314 85.521154) (end 219.791314 74.894) (width 0.2) (layer "F.Cu") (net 4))
 (segment (start 219.791314 72.092) (end 216.802 72.092) (width 0.2) (layer "F.Cu") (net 4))
 (segment (start 214.416634 95.081) (end 220.299634 89.198) (width 0.2) (layer "F.Cu") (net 4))
 (segment (start 219.791314 74.894) (end 220.612 74.073314) (width 0.2) (layer "F.Cu") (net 4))
 (segment (start 205.68331 48.461) (end 212.861 55.63869) (width 0.2) (layer "F.Cu") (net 4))
 (segment (start 212.861 95.081) (end 214.416634 95.081) (width 0.2) (layer "F.Cu") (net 4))
 (segment (start 216.802 72.092) (end 212.861 76.033) (width 0.2) (layer "F.Cu") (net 4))
 (segment (start 221.582 88.88216) (end 221.582 87.31184) (width 0.2) (layer "F.Cu") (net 4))
 (segment (start 220.612 72.912686) (end 219.791314 72.092) (width 0.2) (layer "F.Cu") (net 4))
 (segment (start 212.861 55.63869) (end 212.861 56.985) (width 0.2) (layer "F.Cu") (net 4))
 (segment (start 213.962 58.086) (end 213.962 74.932) (width 0.2) (layer "B.Cu") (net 4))
 (segment (start 212.861 56.985) (end 213.962 58.086) (width 0.2) (layer "B.Cu") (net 4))
 (segment (start 213.962 74.932) (end 212.861 76.033) (width 0.2) (layer "B.Cu") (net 4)))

